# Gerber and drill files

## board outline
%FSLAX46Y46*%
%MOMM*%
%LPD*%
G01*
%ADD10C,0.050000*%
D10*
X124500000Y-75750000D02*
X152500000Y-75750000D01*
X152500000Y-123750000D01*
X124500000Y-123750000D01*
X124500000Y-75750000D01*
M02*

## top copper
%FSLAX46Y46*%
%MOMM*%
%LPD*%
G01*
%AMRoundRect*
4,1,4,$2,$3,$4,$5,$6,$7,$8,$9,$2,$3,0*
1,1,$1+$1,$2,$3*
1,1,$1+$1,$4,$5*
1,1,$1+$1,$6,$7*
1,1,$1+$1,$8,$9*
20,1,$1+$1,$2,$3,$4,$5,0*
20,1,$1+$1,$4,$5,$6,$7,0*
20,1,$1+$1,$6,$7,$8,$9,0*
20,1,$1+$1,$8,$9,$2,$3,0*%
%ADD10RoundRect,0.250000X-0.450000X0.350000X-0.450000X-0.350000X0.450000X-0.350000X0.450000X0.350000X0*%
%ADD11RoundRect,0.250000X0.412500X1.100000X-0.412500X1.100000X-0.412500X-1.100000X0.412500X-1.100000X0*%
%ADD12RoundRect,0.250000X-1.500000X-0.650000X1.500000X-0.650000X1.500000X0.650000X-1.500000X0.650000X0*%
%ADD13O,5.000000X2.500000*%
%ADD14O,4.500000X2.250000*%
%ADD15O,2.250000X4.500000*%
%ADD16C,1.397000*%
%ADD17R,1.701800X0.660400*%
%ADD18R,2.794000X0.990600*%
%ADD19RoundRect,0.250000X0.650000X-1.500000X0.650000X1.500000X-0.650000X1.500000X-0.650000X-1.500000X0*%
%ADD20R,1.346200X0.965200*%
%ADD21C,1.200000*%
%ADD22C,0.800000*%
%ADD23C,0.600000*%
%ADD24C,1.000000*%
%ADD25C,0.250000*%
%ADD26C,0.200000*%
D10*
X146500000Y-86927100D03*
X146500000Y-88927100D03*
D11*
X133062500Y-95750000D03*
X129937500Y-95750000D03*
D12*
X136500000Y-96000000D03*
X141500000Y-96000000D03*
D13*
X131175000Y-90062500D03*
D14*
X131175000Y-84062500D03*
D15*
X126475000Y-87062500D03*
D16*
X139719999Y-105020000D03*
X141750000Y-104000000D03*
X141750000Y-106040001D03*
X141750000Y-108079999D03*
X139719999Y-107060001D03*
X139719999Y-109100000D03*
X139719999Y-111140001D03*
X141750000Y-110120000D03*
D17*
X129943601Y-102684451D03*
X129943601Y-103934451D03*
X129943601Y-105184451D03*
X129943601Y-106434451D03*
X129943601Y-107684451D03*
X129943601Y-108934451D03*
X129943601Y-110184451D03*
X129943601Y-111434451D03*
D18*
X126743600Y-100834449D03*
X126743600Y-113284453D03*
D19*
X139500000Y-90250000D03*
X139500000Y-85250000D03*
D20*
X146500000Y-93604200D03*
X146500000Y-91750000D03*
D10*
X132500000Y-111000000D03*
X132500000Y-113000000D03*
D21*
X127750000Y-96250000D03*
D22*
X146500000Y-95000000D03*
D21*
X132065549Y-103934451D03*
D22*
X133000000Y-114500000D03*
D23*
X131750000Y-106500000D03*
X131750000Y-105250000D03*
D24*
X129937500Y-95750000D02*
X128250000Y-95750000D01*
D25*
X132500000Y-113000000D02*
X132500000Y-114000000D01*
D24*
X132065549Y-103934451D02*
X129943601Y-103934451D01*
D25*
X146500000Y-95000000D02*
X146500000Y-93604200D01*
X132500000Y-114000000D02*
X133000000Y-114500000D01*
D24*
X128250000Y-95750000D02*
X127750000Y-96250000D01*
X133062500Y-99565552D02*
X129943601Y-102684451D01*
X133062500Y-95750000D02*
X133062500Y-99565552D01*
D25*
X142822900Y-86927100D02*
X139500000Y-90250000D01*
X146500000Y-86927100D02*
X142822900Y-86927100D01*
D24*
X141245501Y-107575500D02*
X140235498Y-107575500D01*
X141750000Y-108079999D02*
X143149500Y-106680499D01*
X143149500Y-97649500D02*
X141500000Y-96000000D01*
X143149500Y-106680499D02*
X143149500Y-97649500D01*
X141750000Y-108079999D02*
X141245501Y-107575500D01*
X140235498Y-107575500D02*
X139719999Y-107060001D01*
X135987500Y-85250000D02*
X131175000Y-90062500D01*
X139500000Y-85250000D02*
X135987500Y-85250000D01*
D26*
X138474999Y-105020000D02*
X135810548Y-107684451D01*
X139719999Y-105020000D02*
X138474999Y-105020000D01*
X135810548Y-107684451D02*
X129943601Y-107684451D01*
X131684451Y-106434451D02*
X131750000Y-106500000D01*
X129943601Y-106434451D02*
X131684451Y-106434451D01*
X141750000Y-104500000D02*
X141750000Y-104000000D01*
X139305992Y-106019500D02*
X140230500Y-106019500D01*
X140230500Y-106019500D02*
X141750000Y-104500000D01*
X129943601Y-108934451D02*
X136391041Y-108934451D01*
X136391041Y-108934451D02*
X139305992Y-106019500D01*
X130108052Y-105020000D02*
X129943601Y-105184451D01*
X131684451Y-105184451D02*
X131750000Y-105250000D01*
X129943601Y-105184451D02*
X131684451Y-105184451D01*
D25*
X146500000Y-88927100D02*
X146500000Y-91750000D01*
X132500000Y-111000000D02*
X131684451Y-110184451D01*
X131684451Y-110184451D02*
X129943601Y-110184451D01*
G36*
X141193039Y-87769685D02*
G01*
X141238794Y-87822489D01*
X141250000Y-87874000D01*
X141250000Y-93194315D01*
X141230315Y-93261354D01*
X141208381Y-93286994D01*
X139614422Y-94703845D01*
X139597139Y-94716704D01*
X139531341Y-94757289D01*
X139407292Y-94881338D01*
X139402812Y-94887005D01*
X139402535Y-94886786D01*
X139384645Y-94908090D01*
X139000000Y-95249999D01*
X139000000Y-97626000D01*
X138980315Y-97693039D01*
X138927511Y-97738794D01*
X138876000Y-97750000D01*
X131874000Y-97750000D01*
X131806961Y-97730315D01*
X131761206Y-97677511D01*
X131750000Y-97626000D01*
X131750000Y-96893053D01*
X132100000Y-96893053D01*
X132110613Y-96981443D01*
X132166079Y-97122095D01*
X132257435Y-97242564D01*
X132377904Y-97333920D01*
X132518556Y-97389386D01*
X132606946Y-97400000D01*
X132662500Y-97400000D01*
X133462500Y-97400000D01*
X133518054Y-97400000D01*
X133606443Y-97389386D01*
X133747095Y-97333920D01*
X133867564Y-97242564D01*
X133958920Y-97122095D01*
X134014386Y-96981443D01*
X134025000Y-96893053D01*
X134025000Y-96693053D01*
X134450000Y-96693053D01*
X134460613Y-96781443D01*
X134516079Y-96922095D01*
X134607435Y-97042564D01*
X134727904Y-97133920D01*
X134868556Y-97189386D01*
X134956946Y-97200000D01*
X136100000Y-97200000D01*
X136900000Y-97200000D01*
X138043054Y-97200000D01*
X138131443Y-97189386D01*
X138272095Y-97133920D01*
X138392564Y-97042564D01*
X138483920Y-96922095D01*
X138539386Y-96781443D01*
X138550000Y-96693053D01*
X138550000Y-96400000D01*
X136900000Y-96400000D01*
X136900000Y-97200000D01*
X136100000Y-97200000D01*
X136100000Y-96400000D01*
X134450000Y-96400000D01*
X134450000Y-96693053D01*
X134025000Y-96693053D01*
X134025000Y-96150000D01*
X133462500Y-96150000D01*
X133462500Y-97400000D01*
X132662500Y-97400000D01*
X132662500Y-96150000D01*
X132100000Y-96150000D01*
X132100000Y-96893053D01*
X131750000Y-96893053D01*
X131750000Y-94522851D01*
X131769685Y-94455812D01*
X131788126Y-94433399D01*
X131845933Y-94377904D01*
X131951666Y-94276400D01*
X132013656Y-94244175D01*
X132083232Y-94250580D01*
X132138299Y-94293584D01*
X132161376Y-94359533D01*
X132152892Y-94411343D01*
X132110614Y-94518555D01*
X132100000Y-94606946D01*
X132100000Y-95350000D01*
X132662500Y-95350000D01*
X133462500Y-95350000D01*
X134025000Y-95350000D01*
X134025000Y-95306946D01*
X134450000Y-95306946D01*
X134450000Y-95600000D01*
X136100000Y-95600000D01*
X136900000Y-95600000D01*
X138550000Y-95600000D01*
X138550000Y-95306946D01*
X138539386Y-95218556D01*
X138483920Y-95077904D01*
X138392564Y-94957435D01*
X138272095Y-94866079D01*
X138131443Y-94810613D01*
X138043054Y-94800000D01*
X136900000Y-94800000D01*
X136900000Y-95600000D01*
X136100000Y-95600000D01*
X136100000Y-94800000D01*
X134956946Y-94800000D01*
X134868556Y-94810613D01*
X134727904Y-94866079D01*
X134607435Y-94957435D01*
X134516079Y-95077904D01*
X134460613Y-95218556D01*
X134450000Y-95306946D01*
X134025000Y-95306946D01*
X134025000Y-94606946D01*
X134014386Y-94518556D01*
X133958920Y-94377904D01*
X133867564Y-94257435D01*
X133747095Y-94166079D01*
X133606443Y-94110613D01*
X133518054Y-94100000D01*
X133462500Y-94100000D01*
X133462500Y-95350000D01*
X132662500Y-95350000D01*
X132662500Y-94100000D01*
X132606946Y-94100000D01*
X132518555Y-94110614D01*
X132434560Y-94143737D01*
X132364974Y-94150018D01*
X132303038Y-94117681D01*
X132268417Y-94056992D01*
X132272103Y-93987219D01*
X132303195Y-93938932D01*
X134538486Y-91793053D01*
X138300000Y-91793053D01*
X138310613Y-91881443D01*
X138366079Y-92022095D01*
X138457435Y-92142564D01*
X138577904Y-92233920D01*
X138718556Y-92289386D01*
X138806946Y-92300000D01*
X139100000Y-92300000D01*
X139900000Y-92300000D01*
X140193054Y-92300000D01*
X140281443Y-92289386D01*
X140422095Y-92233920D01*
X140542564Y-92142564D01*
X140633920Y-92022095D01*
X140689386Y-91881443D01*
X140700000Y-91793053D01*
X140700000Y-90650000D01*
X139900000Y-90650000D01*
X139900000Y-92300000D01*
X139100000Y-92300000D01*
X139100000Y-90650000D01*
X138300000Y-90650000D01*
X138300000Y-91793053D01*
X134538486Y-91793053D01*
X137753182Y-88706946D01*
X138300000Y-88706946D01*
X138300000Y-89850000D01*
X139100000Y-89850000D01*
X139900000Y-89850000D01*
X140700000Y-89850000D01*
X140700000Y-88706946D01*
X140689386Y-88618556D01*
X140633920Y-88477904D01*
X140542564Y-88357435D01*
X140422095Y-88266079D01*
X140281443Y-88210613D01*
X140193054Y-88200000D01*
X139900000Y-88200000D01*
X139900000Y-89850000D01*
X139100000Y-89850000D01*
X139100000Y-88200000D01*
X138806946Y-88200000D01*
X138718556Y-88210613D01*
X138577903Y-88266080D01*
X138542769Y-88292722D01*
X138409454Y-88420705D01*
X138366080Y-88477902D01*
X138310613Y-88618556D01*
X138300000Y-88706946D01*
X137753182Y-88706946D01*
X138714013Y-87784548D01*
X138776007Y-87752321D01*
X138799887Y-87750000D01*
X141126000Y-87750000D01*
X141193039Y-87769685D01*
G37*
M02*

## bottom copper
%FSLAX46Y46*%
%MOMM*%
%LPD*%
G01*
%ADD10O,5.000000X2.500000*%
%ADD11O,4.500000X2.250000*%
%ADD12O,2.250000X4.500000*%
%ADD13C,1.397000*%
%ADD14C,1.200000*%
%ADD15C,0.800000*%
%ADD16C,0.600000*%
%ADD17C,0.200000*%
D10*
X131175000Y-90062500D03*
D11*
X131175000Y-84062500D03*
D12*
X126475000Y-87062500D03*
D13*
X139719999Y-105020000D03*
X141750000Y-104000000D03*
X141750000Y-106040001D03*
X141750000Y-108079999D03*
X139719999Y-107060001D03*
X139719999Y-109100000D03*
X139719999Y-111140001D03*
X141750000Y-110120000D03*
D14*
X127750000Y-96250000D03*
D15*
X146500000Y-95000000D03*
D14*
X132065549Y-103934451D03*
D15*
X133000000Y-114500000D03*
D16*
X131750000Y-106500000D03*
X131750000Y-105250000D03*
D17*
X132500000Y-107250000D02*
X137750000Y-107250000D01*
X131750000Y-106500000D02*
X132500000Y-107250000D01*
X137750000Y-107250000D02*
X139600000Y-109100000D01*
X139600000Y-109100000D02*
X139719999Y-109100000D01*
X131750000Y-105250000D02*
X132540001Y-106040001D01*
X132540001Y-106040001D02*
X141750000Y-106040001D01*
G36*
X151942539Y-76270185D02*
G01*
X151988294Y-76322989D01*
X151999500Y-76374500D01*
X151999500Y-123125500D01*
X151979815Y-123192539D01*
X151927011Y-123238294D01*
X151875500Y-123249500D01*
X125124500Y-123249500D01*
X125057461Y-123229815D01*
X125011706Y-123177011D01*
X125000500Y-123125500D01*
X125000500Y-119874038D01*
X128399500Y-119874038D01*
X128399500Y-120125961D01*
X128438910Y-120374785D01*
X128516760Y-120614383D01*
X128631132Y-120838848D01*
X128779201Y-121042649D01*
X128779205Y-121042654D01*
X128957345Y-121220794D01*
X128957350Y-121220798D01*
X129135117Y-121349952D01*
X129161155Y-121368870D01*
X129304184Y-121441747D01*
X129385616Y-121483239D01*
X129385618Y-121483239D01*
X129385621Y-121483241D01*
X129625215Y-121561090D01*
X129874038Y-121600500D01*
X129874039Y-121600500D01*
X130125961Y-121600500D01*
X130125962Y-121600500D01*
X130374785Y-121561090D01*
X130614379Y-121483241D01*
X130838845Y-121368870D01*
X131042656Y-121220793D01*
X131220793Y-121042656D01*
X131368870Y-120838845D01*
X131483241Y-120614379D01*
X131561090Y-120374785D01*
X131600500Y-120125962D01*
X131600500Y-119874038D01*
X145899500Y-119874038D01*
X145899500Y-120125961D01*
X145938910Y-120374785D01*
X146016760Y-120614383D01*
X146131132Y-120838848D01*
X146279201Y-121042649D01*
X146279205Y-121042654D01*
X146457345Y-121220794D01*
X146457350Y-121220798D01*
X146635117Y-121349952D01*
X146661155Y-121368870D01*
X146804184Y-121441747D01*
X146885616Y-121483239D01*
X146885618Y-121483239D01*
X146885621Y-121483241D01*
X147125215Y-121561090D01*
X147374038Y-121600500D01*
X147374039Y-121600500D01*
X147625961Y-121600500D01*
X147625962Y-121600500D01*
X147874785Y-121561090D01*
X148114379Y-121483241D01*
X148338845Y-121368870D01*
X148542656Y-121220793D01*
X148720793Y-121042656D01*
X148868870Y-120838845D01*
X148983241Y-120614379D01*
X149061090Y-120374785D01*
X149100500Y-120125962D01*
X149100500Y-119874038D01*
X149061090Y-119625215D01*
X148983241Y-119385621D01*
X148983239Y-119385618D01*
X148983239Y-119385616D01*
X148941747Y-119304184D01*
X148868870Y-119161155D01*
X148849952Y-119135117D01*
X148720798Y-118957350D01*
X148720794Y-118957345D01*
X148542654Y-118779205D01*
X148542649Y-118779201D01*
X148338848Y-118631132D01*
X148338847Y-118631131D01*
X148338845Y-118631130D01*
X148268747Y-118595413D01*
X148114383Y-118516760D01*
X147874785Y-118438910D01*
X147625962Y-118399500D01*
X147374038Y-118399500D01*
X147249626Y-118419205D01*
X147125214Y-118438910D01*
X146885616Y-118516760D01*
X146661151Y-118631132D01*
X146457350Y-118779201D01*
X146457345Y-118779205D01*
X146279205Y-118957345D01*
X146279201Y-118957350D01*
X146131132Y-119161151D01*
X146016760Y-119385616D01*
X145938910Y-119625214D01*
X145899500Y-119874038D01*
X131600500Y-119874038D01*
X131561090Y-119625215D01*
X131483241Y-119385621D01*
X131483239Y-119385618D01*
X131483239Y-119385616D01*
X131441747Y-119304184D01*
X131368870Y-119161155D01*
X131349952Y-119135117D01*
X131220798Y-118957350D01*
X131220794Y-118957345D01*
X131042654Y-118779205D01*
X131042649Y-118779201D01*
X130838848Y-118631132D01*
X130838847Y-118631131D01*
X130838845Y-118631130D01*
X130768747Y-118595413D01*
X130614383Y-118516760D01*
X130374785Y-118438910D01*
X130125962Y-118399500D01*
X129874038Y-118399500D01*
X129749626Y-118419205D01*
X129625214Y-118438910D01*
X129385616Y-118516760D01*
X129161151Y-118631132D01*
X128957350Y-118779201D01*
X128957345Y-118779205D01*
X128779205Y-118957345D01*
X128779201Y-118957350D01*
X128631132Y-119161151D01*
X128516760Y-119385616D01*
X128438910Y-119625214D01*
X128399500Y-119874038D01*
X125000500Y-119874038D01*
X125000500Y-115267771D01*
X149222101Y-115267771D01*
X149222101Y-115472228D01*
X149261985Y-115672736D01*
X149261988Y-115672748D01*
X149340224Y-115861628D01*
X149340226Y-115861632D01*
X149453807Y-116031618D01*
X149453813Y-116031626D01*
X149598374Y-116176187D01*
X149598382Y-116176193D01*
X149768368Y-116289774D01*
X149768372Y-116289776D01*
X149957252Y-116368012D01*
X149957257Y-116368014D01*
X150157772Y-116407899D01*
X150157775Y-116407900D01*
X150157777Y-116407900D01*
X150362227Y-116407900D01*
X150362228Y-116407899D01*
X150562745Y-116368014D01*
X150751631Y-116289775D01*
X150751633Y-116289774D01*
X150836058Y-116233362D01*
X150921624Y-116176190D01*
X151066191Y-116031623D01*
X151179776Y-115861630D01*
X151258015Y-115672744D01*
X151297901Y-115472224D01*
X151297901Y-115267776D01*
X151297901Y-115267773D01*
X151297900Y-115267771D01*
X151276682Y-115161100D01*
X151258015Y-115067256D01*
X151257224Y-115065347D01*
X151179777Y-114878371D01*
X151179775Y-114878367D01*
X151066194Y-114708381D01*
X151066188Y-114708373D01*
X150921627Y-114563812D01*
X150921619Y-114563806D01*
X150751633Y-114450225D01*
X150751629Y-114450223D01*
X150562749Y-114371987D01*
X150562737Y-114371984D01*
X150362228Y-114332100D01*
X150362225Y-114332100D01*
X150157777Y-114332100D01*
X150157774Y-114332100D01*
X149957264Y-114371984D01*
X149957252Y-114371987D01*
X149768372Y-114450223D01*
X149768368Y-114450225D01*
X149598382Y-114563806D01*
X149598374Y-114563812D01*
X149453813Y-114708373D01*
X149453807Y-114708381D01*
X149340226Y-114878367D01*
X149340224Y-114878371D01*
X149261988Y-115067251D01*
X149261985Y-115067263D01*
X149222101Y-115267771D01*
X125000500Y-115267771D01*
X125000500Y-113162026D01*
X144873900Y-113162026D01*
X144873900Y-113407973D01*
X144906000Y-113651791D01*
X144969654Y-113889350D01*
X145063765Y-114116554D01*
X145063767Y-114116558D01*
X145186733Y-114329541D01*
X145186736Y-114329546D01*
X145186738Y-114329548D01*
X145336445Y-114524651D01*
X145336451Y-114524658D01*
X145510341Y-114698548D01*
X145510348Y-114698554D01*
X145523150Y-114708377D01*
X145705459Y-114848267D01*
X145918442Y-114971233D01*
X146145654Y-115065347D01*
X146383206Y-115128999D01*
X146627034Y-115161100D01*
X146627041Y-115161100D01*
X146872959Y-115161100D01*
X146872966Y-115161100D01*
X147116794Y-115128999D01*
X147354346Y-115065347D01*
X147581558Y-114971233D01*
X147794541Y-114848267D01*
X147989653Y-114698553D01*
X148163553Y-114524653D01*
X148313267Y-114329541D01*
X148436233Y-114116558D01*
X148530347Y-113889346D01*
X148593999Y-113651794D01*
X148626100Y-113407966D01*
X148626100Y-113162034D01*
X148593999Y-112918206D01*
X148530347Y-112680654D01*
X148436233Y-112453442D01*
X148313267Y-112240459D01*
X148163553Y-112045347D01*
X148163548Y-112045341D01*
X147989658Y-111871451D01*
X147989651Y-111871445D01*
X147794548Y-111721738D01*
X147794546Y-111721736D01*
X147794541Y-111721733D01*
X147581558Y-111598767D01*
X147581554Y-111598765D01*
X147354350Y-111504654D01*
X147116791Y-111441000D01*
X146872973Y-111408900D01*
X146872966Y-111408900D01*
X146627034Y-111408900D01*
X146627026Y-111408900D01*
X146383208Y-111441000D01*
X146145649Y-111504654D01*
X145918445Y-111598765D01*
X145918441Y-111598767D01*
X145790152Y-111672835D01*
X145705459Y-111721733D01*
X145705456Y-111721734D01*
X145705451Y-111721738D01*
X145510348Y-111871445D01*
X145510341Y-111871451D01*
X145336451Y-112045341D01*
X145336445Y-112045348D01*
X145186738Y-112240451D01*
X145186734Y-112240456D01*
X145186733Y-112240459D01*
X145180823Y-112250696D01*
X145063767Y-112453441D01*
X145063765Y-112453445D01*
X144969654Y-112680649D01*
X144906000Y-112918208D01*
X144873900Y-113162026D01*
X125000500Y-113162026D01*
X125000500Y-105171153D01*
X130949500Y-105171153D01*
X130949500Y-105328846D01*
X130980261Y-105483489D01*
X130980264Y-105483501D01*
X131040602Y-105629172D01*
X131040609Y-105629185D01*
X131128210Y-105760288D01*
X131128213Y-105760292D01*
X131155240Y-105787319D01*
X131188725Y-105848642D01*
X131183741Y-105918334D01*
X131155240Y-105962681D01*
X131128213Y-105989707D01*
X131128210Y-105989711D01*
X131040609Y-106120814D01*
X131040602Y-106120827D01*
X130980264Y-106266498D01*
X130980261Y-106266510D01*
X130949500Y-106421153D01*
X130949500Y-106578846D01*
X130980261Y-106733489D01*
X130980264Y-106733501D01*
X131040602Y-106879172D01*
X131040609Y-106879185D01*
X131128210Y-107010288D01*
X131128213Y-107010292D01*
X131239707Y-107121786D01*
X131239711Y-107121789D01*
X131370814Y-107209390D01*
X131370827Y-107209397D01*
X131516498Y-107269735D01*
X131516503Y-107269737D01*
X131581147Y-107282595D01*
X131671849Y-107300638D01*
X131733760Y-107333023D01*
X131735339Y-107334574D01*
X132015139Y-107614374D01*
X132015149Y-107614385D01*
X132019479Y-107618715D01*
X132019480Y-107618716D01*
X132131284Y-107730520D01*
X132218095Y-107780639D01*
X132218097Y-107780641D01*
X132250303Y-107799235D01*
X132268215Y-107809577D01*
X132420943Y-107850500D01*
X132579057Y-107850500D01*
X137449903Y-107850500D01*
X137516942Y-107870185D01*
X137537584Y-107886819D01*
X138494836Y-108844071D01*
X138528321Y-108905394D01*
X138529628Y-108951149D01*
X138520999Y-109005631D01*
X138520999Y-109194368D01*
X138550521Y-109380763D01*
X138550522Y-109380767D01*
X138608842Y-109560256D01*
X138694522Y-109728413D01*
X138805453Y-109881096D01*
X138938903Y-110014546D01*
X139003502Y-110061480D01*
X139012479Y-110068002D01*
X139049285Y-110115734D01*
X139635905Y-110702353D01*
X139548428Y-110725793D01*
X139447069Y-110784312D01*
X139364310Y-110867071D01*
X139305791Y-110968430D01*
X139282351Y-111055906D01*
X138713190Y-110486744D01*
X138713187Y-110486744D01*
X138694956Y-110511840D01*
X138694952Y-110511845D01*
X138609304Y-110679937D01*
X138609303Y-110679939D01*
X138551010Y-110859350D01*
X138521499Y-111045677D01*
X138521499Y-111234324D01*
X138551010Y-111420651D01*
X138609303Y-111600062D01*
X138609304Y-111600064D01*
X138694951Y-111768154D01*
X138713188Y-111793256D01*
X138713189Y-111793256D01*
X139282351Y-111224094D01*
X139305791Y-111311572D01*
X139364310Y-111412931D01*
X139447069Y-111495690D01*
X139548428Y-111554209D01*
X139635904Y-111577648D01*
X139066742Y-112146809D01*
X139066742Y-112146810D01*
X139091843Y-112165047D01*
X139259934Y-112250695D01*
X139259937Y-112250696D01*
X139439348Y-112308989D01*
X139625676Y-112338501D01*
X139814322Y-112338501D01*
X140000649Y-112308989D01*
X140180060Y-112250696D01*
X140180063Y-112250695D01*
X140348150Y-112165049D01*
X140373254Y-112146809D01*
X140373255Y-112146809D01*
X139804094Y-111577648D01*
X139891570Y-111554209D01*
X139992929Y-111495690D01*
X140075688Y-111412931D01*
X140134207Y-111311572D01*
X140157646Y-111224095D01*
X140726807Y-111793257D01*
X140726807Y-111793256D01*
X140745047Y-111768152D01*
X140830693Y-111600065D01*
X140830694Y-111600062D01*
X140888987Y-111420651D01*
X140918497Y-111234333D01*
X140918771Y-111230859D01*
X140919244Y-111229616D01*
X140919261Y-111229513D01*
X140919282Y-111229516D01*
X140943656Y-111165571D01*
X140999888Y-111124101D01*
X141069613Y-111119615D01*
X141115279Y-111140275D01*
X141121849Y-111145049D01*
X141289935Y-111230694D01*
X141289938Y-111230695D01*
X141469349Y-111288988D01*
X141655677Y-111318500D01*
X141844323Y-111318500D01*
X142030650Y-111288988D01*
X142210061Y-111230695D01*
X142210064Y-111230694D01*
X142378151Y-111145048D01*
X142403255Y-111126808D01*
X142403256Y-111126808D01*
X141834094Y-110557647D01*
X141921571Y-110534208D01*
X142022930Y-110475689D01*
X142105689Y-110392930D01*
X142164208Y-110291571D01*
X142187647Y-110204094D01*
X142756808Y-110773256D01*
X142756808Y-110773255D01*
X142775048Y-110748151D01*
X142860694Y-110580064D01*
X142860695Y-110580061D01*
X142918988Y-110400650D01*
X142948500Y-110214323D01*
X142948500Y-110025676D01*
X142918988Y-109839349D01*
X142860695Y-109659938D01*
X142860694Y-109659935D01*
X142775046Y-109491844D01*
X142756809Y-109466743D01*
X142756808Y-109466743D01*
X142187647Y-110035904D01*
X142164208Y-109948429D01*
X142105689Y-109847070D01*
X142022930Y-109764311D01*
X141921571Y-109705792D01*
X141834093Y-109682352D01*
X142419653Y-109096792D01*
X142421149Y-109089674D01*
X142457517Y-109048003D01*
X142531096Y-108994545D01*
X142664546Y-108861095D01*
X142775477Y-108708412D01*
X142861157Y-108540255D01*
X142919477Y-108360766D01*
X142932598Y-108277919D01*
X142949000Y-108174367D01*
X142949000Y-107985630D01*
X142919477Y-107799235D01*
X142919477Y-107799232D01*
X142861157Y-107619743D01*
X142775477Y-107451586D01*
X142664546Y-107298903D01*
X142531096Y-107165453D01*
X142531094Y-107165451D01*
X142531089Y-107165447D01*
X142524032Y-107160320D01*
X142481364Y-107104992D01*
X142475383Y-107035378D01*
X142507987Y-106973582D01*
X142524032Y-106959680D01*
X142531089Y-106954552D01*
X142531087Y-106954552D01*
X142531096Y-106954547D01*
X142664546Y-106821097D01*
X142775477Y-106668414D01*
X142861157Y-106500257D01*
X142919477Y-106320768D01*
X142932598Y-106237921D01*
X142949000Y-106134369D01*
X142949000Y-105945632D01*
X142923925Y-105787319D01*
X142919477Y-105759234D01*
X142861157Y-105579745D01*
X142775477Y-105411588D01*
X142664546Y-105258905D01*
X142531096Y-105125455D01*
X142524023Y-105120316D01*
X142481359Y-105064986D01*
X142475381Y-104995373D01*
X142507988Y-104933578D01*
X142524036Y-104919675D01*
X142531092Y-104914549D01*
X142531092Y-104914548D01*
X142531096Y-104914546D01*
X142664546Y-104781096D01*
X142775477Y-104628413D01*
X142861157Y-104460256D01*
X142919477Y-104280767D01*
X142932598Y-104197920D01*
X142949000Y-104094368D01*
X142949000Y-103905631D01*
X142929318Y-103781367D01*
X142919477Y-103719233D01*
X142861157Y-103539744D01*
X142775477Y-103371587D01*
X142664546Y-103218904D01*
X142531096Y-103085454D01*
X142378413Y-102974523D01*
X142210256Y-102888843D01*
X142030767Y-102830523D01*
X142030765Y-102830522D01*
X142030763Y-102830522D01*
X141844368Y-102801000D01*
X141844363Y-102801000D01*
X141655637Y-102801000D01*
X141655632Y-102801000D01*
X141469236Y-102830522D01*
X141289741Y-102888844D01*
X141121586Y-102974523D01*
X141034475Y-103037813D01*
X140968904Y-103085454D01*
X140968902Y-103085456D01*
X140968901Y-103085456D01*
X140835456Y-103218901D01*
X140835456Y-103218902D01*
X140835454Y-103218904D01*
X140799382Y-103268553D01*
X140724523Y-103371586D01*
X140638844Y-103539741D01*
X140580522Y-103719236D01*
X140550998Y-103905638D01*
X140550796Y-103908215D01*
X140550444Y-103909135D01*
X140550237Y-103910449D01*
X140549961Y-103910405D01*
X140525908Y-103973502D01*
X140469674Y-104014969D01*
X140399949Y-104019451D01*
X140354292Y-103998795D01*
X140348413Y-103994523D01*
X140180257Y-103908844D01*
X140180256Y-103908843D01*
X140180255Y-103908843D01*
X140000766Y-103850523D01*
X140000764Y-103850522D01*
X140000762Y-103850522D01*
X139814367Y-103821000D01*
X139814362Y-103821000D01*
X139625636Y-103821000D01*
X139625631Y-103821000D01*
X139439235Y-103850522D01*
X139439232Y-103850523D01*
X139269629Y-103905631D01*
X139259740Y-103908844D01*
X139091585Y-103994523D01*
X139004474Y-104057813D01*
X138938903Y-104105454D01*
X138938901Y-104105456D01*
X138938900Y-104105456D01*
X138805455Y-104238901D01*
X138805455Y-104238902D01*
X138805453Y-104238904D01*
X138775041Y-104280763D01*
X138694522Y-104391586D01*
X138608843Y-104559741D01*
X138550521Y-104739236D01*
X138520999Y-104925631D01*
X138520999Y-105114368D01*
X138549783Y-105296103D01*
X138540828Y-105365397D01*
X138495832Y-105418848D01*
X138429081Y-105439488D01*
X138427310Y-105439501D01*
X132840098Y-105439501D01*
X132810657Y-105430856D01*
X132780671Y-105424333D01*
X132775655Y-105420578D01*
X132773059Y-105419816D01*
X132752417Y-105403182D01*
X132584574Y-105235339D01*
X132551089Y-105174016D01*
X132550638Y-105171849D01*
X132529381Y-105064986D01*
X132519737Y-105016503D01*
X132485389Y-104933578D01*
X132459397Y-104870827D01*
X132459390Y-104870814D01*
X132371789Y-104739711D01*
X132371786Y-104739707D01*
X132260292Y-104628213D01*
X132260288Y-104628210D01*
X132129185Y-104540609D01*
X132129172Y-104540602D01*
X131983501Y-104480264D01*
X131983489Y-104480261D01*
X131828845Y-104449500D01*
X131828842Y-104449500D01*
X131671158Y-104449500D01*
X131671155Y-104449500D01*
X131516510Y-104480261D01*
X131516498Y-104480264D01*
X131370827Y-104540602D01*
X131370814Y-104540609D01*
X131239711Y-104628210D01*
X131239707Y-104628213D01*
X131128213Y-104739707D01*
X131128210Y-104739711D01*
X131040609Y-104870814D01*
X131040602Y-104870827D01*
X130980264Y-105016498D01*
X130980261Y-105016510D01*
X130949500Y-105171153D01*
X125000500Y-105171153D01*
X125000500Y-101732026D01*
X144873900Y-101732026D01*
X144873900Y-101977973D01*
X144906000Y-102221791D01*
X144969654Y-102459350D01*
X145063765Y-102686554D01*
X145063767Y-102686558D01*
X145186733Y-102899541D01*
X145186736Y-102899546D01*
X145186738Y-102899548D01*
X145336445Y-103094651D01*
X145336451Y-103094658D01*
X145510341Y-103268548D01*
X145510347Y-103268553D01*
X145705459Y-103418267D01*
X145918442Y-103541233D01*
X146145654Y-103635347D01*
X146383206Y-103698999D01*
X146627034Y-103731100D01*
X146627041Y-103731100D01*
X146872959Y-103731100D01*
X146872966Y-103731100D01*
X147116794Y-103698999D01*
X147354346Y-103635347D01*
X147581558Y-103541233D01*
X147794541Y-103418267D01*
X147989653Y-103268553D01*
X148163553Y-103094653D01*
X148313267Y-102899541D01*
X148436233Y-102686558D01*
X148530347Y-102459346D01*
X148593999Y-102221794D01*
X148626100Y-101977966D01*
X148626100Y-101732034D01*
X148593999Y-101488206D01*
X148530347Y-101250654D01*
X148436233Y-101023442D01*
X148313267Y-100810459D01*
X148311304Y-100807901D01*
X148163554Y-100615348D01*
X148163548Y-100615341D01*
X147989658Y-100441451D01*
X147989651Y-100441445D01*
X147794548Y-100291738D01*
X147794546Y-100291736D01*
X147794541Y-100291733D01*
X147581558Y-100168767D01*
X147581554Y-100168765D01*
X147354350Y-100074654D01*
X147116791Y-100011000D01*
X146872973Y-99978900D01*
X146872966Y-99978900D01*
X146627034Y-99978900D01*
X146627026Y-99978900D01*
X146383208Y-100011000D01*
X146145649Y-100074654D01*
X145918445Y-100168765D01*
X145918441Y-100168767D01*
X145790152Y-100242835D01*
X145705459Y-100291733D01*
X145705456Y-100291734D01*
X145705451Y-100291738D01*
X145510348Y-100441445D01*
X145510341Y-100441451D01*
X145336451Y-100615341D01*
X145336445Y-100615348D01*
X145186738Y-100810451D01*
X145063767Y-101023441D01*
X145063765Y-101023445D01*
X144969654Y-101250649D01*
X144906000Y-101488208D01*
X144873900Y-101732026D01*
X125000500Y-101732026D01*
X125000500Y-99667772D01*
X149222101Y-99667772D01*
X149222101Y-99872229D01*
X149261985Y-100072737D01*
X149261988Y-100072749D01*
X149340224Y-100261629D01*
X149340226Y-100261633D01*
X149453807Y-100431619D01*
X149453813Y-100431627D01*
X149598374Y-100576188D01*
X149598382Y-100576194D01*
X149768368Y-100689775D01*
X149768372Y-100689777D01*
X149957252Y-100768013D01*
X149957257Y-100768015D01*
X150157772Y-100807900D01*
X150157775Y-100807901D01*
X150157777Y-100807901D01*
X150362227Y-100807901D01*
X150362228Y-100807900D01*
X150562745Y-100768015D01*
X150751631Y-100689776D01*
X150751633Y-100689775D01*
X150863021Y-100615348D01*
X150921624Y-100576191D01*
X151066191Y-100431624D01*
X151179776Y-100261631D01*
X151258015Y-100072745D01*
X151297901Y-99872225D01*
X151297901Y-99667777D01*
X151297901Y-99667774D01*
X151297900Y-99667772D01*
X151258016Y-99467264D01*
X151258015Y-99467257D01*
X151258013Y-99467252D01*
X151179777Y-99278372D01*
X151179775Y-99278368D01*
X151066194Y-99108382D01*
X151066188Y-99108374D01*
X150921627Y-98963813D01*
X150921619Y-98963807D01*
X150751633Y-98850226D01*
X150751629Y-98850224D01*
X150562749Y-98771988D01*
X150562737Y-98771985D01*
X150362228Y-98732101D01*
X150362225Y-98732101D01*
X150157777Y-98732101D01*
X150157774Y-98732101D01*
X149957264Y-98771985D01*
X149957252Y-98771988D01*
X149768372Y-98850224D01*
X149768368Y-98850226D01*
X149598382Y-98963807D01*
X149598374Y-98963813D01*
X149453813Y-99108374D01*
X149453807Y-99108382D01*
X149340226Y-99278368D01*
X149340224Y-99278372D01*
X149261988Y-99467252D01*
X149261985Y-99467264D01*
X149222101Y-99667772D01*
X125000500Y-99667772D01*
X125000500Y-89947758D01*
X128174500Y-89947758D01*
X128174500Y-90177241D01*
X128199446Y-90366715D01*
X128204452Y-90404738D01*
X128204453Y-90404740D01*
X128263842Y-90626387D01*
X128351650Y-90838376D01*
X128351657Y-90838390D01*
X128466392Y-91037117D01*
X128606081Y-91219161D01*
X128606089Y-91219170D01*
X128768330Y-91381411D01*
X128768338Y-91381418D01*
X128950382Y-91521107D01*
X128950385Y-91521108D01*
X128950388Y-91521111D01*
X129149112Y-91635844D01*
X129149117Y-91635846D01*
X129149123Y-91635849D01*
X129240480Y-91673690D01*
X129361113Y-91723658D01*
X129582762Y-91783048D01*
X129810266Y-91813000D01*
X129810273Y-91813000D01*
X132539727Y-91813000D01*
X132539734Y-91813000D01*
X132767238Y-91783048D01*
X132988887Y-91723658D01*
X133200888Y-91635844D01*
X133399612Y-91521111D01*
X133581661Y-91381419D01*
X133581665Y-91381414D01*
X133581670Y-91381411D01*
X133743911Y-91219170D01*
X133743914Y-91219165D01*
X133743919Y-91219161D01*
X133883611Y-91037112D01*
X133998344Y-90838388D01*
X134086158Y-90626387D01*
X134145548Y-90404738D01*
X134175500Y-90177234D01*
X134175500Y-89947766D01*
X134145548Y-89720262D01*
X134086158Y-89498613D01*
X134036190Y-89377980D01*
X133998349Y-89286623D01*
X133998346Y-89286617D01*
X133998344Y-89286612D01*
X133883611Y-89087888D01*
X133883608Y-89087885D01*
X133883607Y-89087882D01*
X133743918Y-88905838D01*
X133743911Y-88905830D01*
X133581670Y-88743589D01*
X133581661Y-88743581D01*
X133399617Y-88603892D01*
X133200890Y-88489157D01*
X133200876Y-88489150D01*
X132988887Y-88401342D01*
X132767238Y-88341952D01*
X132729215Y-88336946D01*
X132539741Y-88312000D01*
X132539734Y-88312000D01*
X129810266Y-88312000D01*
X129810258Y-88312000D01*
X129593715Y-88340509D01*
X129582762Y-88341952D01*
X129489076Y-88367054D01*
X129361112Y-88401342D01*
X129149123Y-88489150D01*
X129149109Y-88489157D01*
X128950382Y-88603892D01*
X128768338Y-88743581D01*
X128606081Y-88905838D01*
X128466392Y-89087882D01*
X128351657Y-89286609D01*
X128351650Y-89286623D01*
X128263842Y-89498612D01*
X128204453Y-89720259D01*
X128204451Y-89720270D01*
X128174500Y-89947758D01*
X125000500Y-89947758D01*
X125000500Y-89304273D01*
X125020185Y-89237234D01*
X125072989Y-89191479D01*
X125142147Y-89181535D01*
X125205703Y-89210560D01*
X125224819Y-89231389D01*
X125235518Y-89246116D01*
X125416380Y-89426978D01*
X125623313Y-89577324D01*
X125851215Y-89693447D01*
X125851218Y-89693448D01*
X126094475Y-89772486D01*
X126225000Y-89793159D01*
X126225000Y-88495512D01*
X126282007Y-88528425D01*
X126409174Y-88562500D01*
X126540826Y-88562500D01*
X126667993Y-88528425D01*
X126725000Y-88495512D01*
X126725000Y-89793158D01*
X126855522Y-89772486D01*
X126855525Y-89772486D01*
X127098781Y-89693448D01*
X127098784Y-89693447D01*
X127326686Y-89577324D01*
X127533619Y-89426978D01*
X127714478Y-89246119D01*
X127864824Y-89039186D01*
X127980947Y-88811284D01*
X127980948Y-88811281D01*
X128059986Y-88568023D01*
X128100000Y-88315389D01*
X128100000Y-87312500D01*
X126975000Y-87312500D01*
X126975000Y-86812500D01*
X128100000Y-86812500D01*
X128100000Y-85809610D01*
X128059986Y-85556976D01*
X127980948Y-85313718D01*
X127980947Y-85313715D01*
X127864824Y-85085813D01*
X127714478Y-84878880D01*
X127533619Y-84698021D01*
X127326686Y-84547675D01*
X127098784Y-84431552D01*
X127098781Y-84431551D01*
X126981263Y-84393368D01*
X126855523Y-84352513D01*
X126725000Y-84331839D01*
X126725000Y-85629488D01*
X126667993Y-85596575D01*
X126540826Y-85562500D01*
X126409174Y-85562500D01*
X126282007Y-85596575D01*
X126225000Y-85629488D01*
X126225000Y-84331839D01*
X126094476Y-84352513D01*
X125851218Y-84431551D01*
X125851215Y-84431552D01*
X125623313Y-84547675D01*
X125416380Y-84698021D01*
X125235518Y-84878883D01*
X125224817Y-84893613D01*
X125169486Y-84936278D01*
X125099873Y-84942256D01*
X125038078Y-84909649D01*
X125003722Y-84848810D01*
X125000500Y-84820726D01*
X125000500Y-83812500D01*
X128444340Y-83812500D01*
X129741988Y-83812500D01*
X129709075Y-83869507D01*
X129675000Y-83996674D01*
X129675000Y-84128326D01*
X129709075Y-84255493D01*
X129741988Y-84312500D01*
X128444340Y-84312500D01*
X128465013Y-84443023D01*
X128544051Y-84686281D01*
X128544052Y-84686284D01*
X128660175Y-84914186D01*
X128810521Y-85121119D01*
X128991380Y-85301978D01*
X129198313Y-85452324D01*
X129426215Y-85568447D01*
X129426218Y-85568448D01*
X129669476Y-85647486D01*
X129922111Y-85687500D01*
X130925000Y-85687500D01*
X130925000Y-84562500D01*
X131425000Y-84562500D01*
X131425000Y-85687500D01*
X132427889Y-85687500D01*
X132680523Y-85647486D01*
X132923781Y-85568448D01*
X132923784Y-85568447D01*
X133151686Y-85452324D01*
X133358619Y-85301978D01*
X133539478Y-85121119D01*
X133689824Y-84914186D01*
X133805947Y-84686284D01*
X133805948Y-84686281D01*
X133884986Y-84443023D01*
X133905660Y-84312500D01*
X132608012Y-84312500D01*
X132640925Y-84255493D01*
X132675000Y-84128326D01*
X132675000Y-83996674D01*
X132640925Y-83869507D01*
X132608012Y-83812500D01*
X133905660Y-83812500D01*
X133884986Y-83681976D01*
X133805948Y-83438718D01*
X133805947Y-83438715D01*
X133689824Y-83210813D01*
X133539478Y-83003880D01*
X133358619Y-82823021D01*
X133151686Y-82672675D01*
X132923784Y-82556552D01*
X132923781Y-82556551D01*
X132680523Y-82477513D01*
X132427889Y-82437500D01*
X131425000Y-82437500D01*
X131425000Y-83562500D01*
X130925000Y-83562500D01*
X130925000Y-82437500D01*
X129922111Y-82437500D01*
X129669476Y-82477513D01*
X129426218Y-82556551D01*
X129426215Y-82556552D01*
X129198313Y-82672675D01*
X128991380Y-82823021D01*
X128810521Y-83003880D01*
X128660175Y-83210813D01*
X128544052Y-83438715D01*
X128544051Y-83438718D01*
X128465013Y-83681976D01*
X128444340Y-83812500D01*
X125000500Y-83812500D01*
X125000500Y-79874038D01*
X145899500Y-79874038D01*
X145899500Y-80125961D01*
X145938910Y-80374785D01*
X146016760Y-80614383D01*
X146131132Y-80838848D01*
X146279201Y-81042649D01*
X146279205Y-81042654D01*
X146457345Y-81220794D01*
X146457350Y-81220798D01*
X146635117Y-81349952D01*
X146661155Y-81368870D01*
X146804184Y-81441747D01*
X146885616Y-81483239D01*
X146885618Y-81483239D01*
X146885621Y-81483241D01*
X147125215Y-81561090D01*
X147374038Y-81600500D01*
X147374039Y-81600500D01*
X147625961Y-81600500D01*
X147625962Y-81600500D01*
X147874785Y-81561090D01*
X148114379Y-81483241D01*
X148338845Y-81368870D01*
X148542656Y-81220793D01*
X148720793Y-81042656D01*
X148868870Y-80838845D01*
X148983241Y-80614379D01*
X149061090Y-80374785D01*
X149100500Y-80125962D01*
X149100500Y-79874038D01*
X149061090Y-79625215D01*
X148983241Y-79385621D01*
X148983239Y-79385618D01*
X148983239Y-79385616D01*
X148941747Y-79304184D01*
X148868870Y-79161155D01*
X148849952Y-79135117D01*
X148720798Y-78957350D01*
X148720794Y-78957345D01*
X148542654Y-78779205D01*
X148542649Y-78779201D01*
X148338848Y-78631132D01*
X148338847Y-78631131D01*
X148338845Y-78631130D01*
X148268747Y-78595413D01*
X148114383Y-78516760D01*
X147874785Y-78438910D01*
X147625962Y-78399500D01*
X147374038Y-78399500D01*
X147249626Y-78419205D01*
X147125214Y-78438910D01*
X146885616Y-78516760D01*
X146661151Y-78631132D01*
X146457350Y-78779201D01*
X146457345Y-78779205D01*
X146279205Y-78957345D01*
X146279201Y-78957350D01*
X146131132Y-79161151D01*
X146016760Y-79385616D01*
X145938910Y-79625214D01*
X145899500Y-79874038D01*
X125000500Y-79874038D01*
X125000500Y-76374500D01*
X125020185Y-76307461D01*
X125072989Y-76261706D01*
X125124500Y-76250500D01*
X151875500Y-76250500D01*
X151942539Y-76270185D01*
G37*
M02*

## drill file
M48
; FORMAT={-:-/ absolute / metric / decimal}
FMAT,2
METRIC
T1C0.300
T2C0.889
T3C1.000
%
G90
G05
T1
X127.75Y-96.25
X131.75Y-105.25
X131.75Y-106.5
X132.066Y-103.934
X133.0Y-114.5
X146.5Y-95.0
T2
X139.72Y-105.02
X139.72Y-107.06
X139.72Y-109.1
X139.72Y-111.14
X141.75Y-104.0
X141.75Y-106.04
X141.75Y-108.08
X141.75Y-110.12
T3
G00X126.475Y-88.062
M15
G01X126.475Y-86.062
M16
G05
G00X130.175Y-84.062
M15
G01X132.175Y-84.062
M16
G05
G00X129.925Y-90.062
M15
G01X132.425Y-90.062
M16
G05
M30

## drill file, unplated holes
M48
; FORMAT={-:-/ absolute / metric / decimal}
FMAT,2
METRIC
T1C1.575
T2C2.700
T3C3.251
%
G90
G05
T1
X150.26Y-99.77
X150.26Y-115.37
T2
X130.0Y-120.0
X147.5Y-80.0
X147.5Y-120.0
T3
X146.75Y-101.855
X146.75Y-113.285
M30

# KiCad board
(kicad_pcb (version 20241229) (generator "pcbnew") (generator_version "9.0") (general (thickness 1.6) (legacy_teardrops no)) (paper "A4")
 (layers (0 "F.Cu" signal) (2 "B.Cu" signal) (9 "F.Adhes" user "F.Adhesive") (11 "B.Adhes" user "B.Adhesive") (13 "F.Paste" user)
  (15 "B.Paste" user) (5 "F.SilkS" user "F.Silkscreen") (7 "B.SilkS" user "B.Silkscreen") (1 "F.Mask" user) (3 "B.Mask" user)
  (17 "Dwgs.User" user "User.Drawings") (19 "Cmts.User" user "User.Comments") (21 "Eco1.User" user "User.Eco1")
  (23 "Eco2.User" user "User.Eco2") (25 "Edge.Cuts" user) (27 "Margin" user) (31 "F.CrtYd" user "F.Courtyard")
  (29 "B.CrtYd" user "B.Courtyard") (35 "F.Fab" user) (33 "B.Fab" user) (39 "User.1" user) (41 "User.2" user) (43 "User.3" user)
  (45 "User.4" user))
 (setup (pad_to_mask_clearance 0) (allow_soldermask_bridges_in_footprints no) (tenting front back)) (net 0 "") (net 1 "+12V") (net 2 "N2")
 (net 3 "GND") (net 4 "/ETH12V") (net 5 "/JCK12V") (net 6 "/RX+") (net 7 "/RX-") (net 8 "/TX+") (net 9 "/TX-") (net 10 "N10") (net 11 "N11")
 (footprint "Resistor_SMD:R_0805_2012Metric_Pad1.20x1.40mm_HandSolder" (layer "F.Cu") (at 146.5 87.9271 -90)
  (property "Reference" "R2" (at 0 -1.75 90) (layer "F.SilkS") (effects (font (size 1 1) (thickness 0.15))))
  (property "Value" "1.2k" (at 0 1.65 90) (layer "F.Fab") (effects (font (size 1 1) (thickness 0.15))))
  (pad "1" smd roundrect (at -1 0 270) (size 1.2 1.4) (layers "F.Cu" "F.Mask" "F.Paste") (roundrect_rratio 0.208333) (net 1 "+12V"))
  (pad "2" smd roundrect (at 1 0 270) (size 1.2 1.4) (layers "F.Cu" "F.Mask" "F.Paste") (roundrect_rratio 0.208333) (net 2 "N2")))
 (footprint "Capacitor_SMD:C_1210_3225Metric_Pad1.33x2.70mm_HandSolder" (layer "F.Cu") (at 131.5 95.75 180)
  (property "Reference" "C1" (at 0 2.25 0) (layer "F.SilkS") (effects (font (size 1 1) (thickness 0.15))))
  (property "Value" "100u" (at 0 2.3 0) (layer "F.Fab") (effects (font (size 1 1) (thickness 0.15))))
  (pad "1" smd roundrect (at -1.5625 0 180) (size 1.325 2.7) (layers "F.Cu" "F.Mask" "F.Paste") (roundrect_rratio 0.188679) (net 1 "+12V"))
  (pad "2" smd roundrect (at 1.5625 0 180) (size 1.325 2.7) (layers "F.Cu" "F.Mask" "F.Paste") (roundrect_rratio 0.188679) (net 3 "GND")))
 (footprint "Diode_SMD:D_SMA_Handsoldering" (layer "F.Cu") (at 139 96)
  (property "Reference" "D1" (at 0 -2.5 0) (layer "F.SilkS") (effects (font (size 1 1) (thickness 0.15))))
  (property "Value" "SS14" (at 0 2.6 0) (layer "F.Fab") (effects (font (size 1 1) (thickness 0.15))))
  (pad "1" smd roundrect (at -2.5 0) (size 3.5 1.8) (layers "F.Cu" "F.Mask" "F.Paste") (roundrect_rratio 0.1388888889) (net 1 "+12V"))
  (pad "2" smd roundrect (at 2.5 0) (size 3.5 1.8) (layers "F.Cu" "F.Mask" "F.Paste") (roundrect_rratio 0.1388888889) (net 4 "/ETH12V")))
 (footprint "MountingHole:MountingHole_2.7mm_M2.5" (layer "F.Cu") (at 130 120)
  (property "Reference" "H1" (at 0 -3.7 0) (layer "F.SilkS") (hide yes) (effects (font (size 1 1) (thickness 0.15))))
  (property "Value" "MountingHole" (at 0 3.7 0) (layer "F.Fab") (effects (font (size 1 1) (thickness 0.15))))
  (pad "" np_thru_hole circle (at 0 0) (size 2.7 2.7) (drill 2.7) (layers "*.Cu" "*.Mask")))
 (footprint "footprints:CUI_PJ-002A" (layer "F.Cu") (at 131.175 90.0625 90)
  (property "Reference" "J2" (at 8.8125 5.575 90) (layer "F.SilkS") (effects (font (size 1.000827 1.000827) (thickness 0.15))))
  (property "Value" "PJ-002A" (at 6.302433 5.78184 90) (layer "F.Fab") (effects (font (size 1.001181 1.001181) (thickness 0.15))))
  (pad "1" thru_hole oval (at 0 0 90) (size 2.5 5) (drill oval 1 3.5) (layers "*.Cu" "*.Mask") (remove_unused_layers no) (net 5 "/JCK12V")
   (solder_mask_margin 0.102))
  (pad "2" thru_hole oval (at 6 0 90) (size 2.25 4.5) (drill oval 1 3) (layers "*.Cu" "*.Mask") (remove_unused_layers no) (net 3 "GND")
   (solder_mask_margin 0.102))
  (pad "3" thru_hole oval (at 3 -4.7 90) (size 4.5 2.25) (drill oval 3 1) (layers "*.Cu" "*.Mask") (remove_unused_layers no) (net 3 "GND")
   (solder_mask_margin 0.102)))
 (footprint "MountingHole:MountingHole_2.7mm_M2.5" (layer "F.Cu") (at 147.5 120)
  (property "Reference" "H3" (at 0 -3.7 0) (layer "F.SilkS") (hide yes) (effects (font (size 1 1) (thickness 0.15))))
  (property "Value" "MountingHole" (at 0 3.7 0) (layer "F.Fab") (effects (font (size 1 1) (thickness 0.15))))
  (pad "" np_thru_hole circle (at 0 0) (size 2.7 2.7) (drill 2.7) (layers "*.Cu" "*.Mask")))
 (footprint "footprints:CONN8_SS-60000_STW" (layer "F.Cu") (at 141.75 104 90)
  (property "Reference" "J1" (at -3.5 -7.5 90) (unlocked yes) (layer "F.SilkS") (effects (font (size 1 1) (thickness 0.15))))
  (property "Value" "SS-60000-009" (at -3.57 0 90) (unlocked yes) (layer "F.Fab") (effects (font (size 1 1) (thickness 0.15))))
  (pad "" np_thru_hole circle (at -11.37 8.510001 90) (size 1.5748 1.5748) (drill 1.5748) (layers))
  (pad "" np_thru_hole circle (at -9.285 5 90) (size 3.2512 3.2512) (drill 3.2512) (layers "*.Cu" "*.Mask"))
  (pad "" np_thru_hole circle (at 2.145 5 90) (size 3.2512 3.2512) (drill 3.2512) (layers "*.Cu" "*.Mask"))
  (pad "" np_thru_hole circle (at 4.229999 8.510001 90) (size 1.5748 1.5748) (drill 1.5748) (layers))
  (pad "1" thru_hole circle (at -1.02 -2.030001 90) (size 1.397 1.397) (drill 0.889) (layers "*.Cu" "*.Mask") (remove_unused_layers no)
   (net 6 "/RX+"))
  (pad "2" thru_hole circle (at 0 0 90) (size 1.397 1.397) (drill 0.889) (layers "*.Cu" "*.Mask") (remove_unused_layers no) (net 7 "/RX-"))
  (pad "3" thru_hole circle (at -2.040001 0 90) (size 1.397 1.397) (drill 0.889) (layers "*.Cu" "*.Mask") (remove_unused_layers no)
   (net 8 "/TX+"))
  (pad "4" thru_hole circle (at -4.079999 0 90) (size 1.397 1.397) (drill 0.889) (layers "*.Cu" "*.Mask") (remove_unused_layers no)
   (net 4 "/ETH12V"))
  (pad "5" thru_hole circle (at -3.060001 -2.030001 90) (size 1.397 1.397) (drill 0.889) (layers "*.Cu" "*.Mask") (remove_unused_layers no)
   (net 4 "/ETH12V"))
  (pad "6" thru_hole circle (at -5.1 -2.030001 90) (size 1.397 1.397) (drill 0.889) (layers "*.Cu" "*.Mask") (remove_unused_layers no)
   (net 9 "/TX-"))
  (pad "7" thru_hole circle (at -7.140001 -2.030001 90) (size 1.397 1.397) (drill 0.889) (layers "*.Cu" "*.Mask") (remove_unused_layers no)
   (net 3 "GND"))
  (pad "8" thru_hole circle (at -6.12 0 90) (size 1.397 1.397) (drill 0.889) (layers "*.Cu" "*.Mask") (remove_unused_layers no)
   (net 3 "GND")))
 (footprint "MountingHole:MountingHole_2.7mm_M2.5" (layer "F.Cu") (at 147.5 80)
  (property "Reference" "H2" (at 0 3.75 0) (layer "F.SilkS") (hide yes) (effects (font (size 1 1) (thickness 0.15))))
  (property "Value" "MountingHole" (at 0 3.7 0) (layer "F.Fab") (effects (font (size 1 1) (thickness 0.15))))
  (pad "" np_thru_hole circle (at 0 0) (size 2.7 2.7) (drill 2.7) (layers "*.Cu" "*.Mask")))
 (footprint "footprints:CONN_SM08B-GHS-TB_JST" (layer "F.Cu") (at 128.067901 107.059451 -90)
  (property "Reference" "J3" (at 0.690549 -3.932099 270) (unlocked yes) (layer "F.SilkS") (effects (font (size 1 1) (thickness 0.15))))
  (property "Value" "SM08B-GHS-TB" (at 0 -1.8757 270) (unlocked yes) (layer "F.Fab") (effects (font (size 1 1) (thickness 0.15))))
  (pad "1" smd rect (at -4.375 -1.8757 270) (size 0.6604 1.7018) (layers "F.Cu" "F.Mask" "F.Paste") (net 1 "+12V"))
  (pad "2" smd rect (at -3.125 -1.8757 270) (size 0.6604 1.7018) (layers "F.Cu" "F.Mask" "F.Paste") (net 3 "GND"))
  (pad "3" smd rect (at -1.875 -1.8757 270) (size 0.6604 1.7018) (layers "F.Cu" "F.Mask" "F.Paste") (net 8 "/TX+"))
  (pad "4" smd rect (at -0.625 -1.8757 270) (size 0.6604 1.7018) (layers "F.Cu" "F.Mask" "F.Paste") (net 9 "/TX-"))
  (pad "5" smd rect (at 0.625 -1.8757 270) (size 0.6604 1.7018) (layers "F.Cu" "F.Mask" "F.Paste") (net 6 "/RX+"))
  (pad "6" smd rect (at 1.875 -1.8757 270) (size 0.6604 1.7018) (layers "F.Cu" "F.Mask" "F.Paste") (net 7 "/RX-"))
  (pad "7" smd rect (at 3.125 -1.8757 270) (size 0.6604 1.7018) (layers "F.Cu" "F.Mask" "F.Paste") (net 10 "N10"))
  (pad "8" smd rect (at 4.375 -1.8757 270) (size 0.6604 1.7018) (layers "F.Cu" "F.Mask" "F.Paste") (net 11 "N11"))
  (pad "9" smd rect (at -6.225002 1.324301 270) (size 0.9906 2.794) (layers "F.Cu" "F.Mask" "F.Paste"))
  (pad "10" smd rect (at 6.225002 1.324301 270) (size 0.9906 2.794) (layers "F.Cu" "F.Mask" "F.Paste")))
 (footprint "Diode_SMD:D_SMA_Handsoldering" (layer "F.Cu") (at 139.5 87.75 90)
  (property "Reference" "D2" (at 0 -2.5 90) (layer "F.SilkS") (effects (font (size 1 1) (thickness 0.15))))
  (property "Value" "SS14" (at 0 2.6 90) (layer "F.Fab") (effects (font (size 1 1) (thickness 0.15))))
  (pad "1" smd roundrect (at -2.5 0 90) (size 3.5 1.8) (layers "F.Cu" "F.Mask" "F.Paste") (roundrect_rratio 0.1388888889) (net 1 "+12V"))
  (pad "2" smd roundrect (at 2.5 0 90) (size 3.5 1.8) (layers "F.Cu" "F.Mask" "F.Paste") (roundrect_rratio 0.1388888889) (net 5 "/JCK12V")))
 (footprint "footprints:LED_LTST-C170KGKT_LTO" (layer "F.Cu") (at 146.5 92.6771 90)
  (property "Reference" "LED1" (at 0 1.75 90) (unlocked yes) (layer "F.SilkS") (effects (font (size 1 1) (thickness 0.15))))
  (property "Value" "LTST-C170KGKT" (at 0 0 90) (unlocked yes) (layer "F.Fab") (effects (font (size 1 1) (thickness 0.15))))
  (pad "1" smd rect (at -0.9271 0 90) (size 0.9652 1.3462) (layers "F.Cu" "F.Mask" "F.Paste") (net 3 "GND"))
  (pad "2" smd rect (at 0.9271 0 90) (size 0.9652 1.3462) (layers "F.Cu" "F.Mask" "F.Paste") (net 2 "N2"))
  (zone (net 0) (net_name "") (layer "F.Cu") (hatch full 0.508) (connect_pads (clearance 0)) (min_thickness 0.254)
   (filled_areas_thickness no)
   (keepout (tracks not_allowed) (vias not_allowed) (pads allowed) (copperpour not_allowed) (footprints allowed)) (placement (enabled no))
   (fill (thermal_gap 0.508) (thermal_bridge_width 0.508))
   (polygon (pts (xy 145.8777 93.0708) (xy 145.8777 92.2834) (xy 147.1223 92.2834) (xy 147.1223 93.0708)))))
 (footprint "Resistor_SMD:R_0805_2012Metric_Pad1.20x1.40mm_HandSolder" (layer "F.Cu") (at 132.5 112 -90)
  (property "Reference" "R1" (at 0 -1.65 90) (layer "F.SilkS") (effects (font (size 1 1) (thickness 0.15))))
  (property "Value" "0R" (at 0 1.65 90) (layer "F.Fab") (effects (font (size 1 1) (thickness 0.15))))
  (pad "1" smd roundrect (at -1 0 270) (size 1.2 1.4) (layers "F.Cu" "F.Mask" "F.Paste") (roundrect_rratio 0.208333) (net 10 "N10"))
  (pad "2" smd roundrect (at 1 0 270) (size 1.2 1.4) (layers "F.Cu" "F.Mask" "F.Paste") (roundrect_rratio 0.208333) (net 3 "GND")))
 (gr_rect (start 124.5 75.75) (end 152.5 123.75) (stroke (width 0.05) (type default)) (fill no) (layer "Edge.Cuts"))
 (segment (start 129.9375 95.75) (end 128.25 95.75) (width 1) (layer "F.Cu") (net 3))
 (segment (start 132.5 113) (end 132.5 114) (width 0.25) (layer "F.Cu") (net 3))
 (segment (start 132.065549 103.934451) (end 129.943601 103.934451) (width 1) (layer "F.Cu") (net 3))
 (segment (start 146.5 95) (end 146.5 93.6042) (width 0.25) (layer "F.Cu") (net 3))
 (segment (start 132.5 114) (end 133 114.5) (width 0.25) (layer "F.Cu") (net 3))
 (segment (start 128.25 95.75) (end 127.75 96.25) (width 1) (layer "F.Cu") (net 3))
 (via (at 127.75 96.25) (size 1.2) (drill 0.3) (layers "F.Cu" "B.Cu") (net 3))
 (via (at 146.5 95) (size 0.8) (drill 0.3) (layers "F.Cu" "B.Cu") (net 3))
 (via (at 132.065549 103.934451) (size 1.2) (drill 0.3) (layers "F.Cu" "B.Cu") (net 3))
 (via (at 133 114.5) (size 0.8) (drill 0.3) (layers "F.Cu" "B.Cu") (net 3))
 (segment (start 133.0625 99.565552) (end 129.943601 102.684451) (width 1) (layer "F.Cu") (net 1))
 (segment (start 133.0625 95.75) (end 133.0625 99.565552) (width 1) (layer "F.Cu") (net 1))
 (segment (start 142.8229 86.9271) (end 139.5 90.25) (width 0.25) (layer "F.Cu") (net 1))
 (segment (start 146.5 86.9271) (end 142.8229 86.9271) (width 0.25) (layer "F.Cu") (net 1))
 (segment (start 141.245501 107.5755) (end 140.235498 107.5755) (width 1) (layer "F.Cu") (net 4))
 (segment (start 141.75 108.079999) (end 143.1495 106.680499) (width 1) (layer "F.Cu") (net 4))
 (segment (start 143.1495 97.6495) (end 141.5 96) (width 1) (layer "F.Cu") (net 4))
 (segment (start 143.1495 106.680499) (end 143.1495 97.6495) (width 1) (layer "F.Cu") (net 4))
 (segment (start 141.75 108.079999) (end 141.245501 107.5755) (width 1) (layer "F.Cu") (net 4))
 (segment (start 140.235498 107.5755) (end 139.719999 107.060001) (width 1) (layer "F.Cu") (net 4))
 (segment (start 135.9875 85.25) (end 131.175 90.0625) (width 1) (layer "F.Cu") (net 5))
 (segment (start 139.5 85.25) (end 135.9875 85.25) (width 1) (layer "F.Cu") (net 5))
 (segment (start 138.474999 105.02) (end 135.810548 107.684451) (width 0.2) (layer "F.Cu") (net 6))
 (segment (start 139.719999 105.02) (end 138.474999 105.02) (width 0.2) (layer "F.Cu") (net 6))
 (segment (start 135.810548 107.684451) (end 129.943601 107.684451) (width 0.2) (layer "F.Cu") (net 6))
 (segment (start 131.684451 106.434451) (end 131.75 106.5) (width 0.2) (layer "F.Cu") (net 9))
 (segment (start 129.943601 106.434451) (end 131.684451 106.434451) (width 0.2) (layer "F.Cu") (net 9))
 (via (at 131.75 106.5) (size 0.6) (drill 0.3) (layers "F.Cu" "B.Cu") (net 9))
 (segment (start 132.5 107.25) (end 137.75 107.25) (width 0.2) (layer "B.Cu") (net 9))
 (segment (start 131.75 106.5) (end 132.5 107.25) (width 0.2) (layer "B.Cu") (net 9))
 (segment (start 137.75 107.25) (end 139.6 109.1) (width 0.2) (layer "B.Cu") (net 9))
 (segment (start 139.6 109.1) (end 139.719999 109.1) (width 0.2) (layer "B.Cu") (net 9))
 (segment (start 141.75 104.5) (end 141.75 104) (width 0.2) (layer "F.Cu") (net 7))
 (segment (start 139.305992 106.0195) (end 140.2305 106.0195) (width 0.2) (layer "F.Cu") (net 7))
 (segment (start 140.2305 106.0195) (end 141.75 104.5) (width 0.2) (layer "F.Cu") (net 7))
 (segment (start 129.943601 108.934451) (end 136.391041 108.934451) (width 0.2) (layer "F.Cu") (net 7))
 (segment (start 136.391041 108.934451) (end 139.305992 106.0195) (width 0.2) (layer "F.Cu") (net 7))
 (segment (start 130.108052 105.02) (end 129.943601 105.184451) (width 0.2) (layer "F.Cu") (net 8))
 (segment (start 131.684451 105.184451) (end 131.75 105.25) (width 0.2) (layer "F.Cu") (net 8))
 (segment (start 129.943601 105.184451) (end 131.684451 105.184451) (width 0.2) (layer "F.Cu") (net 8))
 (via (at 131.75 105.25) (size 0.6) (drill 0.3) (layers "F.Cu" "B.Cu") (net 8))
 (segment (start 131.75 105.25) (end 132.540001 106.040001) (width 0.2) (layer "B.Cu") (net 8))
 (segment (start 132.540001 106.040001) (end 141.75 106.040001) (width 0.2) (layer "B.Cu") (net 8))
 (segment (start 146.5 88.9271) (end 146.5 91.75) (width 0.25) (layer "F.Cu") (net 2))
 (segment (start 132.5 111) (end 131.684451 110.184451) (width 0.25) (layer "F.Cu") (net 10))
 (segment (start 131.684451 110.184451) (end 129.943601 110.184451) (width 0.25) (layer "F.Cu") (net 10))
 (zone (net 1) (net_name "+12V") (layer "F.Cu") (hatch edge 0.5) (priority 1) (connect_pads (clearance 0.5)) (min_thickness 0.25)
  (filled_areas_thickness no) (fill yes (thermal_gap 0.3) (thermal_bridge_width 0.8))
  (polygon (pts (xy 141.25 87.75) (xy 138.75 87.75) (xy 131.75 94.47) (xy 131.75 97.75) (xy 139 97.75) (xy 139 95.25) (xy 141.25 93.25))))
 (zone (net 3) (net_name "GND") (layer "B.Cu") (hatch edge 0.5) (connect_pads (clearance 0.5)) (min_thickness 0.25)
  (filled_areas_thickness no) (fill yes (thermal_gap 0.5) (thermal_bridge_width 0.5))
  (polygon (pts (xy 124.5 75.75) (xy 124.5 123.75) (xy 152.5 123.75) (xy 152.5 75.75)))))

